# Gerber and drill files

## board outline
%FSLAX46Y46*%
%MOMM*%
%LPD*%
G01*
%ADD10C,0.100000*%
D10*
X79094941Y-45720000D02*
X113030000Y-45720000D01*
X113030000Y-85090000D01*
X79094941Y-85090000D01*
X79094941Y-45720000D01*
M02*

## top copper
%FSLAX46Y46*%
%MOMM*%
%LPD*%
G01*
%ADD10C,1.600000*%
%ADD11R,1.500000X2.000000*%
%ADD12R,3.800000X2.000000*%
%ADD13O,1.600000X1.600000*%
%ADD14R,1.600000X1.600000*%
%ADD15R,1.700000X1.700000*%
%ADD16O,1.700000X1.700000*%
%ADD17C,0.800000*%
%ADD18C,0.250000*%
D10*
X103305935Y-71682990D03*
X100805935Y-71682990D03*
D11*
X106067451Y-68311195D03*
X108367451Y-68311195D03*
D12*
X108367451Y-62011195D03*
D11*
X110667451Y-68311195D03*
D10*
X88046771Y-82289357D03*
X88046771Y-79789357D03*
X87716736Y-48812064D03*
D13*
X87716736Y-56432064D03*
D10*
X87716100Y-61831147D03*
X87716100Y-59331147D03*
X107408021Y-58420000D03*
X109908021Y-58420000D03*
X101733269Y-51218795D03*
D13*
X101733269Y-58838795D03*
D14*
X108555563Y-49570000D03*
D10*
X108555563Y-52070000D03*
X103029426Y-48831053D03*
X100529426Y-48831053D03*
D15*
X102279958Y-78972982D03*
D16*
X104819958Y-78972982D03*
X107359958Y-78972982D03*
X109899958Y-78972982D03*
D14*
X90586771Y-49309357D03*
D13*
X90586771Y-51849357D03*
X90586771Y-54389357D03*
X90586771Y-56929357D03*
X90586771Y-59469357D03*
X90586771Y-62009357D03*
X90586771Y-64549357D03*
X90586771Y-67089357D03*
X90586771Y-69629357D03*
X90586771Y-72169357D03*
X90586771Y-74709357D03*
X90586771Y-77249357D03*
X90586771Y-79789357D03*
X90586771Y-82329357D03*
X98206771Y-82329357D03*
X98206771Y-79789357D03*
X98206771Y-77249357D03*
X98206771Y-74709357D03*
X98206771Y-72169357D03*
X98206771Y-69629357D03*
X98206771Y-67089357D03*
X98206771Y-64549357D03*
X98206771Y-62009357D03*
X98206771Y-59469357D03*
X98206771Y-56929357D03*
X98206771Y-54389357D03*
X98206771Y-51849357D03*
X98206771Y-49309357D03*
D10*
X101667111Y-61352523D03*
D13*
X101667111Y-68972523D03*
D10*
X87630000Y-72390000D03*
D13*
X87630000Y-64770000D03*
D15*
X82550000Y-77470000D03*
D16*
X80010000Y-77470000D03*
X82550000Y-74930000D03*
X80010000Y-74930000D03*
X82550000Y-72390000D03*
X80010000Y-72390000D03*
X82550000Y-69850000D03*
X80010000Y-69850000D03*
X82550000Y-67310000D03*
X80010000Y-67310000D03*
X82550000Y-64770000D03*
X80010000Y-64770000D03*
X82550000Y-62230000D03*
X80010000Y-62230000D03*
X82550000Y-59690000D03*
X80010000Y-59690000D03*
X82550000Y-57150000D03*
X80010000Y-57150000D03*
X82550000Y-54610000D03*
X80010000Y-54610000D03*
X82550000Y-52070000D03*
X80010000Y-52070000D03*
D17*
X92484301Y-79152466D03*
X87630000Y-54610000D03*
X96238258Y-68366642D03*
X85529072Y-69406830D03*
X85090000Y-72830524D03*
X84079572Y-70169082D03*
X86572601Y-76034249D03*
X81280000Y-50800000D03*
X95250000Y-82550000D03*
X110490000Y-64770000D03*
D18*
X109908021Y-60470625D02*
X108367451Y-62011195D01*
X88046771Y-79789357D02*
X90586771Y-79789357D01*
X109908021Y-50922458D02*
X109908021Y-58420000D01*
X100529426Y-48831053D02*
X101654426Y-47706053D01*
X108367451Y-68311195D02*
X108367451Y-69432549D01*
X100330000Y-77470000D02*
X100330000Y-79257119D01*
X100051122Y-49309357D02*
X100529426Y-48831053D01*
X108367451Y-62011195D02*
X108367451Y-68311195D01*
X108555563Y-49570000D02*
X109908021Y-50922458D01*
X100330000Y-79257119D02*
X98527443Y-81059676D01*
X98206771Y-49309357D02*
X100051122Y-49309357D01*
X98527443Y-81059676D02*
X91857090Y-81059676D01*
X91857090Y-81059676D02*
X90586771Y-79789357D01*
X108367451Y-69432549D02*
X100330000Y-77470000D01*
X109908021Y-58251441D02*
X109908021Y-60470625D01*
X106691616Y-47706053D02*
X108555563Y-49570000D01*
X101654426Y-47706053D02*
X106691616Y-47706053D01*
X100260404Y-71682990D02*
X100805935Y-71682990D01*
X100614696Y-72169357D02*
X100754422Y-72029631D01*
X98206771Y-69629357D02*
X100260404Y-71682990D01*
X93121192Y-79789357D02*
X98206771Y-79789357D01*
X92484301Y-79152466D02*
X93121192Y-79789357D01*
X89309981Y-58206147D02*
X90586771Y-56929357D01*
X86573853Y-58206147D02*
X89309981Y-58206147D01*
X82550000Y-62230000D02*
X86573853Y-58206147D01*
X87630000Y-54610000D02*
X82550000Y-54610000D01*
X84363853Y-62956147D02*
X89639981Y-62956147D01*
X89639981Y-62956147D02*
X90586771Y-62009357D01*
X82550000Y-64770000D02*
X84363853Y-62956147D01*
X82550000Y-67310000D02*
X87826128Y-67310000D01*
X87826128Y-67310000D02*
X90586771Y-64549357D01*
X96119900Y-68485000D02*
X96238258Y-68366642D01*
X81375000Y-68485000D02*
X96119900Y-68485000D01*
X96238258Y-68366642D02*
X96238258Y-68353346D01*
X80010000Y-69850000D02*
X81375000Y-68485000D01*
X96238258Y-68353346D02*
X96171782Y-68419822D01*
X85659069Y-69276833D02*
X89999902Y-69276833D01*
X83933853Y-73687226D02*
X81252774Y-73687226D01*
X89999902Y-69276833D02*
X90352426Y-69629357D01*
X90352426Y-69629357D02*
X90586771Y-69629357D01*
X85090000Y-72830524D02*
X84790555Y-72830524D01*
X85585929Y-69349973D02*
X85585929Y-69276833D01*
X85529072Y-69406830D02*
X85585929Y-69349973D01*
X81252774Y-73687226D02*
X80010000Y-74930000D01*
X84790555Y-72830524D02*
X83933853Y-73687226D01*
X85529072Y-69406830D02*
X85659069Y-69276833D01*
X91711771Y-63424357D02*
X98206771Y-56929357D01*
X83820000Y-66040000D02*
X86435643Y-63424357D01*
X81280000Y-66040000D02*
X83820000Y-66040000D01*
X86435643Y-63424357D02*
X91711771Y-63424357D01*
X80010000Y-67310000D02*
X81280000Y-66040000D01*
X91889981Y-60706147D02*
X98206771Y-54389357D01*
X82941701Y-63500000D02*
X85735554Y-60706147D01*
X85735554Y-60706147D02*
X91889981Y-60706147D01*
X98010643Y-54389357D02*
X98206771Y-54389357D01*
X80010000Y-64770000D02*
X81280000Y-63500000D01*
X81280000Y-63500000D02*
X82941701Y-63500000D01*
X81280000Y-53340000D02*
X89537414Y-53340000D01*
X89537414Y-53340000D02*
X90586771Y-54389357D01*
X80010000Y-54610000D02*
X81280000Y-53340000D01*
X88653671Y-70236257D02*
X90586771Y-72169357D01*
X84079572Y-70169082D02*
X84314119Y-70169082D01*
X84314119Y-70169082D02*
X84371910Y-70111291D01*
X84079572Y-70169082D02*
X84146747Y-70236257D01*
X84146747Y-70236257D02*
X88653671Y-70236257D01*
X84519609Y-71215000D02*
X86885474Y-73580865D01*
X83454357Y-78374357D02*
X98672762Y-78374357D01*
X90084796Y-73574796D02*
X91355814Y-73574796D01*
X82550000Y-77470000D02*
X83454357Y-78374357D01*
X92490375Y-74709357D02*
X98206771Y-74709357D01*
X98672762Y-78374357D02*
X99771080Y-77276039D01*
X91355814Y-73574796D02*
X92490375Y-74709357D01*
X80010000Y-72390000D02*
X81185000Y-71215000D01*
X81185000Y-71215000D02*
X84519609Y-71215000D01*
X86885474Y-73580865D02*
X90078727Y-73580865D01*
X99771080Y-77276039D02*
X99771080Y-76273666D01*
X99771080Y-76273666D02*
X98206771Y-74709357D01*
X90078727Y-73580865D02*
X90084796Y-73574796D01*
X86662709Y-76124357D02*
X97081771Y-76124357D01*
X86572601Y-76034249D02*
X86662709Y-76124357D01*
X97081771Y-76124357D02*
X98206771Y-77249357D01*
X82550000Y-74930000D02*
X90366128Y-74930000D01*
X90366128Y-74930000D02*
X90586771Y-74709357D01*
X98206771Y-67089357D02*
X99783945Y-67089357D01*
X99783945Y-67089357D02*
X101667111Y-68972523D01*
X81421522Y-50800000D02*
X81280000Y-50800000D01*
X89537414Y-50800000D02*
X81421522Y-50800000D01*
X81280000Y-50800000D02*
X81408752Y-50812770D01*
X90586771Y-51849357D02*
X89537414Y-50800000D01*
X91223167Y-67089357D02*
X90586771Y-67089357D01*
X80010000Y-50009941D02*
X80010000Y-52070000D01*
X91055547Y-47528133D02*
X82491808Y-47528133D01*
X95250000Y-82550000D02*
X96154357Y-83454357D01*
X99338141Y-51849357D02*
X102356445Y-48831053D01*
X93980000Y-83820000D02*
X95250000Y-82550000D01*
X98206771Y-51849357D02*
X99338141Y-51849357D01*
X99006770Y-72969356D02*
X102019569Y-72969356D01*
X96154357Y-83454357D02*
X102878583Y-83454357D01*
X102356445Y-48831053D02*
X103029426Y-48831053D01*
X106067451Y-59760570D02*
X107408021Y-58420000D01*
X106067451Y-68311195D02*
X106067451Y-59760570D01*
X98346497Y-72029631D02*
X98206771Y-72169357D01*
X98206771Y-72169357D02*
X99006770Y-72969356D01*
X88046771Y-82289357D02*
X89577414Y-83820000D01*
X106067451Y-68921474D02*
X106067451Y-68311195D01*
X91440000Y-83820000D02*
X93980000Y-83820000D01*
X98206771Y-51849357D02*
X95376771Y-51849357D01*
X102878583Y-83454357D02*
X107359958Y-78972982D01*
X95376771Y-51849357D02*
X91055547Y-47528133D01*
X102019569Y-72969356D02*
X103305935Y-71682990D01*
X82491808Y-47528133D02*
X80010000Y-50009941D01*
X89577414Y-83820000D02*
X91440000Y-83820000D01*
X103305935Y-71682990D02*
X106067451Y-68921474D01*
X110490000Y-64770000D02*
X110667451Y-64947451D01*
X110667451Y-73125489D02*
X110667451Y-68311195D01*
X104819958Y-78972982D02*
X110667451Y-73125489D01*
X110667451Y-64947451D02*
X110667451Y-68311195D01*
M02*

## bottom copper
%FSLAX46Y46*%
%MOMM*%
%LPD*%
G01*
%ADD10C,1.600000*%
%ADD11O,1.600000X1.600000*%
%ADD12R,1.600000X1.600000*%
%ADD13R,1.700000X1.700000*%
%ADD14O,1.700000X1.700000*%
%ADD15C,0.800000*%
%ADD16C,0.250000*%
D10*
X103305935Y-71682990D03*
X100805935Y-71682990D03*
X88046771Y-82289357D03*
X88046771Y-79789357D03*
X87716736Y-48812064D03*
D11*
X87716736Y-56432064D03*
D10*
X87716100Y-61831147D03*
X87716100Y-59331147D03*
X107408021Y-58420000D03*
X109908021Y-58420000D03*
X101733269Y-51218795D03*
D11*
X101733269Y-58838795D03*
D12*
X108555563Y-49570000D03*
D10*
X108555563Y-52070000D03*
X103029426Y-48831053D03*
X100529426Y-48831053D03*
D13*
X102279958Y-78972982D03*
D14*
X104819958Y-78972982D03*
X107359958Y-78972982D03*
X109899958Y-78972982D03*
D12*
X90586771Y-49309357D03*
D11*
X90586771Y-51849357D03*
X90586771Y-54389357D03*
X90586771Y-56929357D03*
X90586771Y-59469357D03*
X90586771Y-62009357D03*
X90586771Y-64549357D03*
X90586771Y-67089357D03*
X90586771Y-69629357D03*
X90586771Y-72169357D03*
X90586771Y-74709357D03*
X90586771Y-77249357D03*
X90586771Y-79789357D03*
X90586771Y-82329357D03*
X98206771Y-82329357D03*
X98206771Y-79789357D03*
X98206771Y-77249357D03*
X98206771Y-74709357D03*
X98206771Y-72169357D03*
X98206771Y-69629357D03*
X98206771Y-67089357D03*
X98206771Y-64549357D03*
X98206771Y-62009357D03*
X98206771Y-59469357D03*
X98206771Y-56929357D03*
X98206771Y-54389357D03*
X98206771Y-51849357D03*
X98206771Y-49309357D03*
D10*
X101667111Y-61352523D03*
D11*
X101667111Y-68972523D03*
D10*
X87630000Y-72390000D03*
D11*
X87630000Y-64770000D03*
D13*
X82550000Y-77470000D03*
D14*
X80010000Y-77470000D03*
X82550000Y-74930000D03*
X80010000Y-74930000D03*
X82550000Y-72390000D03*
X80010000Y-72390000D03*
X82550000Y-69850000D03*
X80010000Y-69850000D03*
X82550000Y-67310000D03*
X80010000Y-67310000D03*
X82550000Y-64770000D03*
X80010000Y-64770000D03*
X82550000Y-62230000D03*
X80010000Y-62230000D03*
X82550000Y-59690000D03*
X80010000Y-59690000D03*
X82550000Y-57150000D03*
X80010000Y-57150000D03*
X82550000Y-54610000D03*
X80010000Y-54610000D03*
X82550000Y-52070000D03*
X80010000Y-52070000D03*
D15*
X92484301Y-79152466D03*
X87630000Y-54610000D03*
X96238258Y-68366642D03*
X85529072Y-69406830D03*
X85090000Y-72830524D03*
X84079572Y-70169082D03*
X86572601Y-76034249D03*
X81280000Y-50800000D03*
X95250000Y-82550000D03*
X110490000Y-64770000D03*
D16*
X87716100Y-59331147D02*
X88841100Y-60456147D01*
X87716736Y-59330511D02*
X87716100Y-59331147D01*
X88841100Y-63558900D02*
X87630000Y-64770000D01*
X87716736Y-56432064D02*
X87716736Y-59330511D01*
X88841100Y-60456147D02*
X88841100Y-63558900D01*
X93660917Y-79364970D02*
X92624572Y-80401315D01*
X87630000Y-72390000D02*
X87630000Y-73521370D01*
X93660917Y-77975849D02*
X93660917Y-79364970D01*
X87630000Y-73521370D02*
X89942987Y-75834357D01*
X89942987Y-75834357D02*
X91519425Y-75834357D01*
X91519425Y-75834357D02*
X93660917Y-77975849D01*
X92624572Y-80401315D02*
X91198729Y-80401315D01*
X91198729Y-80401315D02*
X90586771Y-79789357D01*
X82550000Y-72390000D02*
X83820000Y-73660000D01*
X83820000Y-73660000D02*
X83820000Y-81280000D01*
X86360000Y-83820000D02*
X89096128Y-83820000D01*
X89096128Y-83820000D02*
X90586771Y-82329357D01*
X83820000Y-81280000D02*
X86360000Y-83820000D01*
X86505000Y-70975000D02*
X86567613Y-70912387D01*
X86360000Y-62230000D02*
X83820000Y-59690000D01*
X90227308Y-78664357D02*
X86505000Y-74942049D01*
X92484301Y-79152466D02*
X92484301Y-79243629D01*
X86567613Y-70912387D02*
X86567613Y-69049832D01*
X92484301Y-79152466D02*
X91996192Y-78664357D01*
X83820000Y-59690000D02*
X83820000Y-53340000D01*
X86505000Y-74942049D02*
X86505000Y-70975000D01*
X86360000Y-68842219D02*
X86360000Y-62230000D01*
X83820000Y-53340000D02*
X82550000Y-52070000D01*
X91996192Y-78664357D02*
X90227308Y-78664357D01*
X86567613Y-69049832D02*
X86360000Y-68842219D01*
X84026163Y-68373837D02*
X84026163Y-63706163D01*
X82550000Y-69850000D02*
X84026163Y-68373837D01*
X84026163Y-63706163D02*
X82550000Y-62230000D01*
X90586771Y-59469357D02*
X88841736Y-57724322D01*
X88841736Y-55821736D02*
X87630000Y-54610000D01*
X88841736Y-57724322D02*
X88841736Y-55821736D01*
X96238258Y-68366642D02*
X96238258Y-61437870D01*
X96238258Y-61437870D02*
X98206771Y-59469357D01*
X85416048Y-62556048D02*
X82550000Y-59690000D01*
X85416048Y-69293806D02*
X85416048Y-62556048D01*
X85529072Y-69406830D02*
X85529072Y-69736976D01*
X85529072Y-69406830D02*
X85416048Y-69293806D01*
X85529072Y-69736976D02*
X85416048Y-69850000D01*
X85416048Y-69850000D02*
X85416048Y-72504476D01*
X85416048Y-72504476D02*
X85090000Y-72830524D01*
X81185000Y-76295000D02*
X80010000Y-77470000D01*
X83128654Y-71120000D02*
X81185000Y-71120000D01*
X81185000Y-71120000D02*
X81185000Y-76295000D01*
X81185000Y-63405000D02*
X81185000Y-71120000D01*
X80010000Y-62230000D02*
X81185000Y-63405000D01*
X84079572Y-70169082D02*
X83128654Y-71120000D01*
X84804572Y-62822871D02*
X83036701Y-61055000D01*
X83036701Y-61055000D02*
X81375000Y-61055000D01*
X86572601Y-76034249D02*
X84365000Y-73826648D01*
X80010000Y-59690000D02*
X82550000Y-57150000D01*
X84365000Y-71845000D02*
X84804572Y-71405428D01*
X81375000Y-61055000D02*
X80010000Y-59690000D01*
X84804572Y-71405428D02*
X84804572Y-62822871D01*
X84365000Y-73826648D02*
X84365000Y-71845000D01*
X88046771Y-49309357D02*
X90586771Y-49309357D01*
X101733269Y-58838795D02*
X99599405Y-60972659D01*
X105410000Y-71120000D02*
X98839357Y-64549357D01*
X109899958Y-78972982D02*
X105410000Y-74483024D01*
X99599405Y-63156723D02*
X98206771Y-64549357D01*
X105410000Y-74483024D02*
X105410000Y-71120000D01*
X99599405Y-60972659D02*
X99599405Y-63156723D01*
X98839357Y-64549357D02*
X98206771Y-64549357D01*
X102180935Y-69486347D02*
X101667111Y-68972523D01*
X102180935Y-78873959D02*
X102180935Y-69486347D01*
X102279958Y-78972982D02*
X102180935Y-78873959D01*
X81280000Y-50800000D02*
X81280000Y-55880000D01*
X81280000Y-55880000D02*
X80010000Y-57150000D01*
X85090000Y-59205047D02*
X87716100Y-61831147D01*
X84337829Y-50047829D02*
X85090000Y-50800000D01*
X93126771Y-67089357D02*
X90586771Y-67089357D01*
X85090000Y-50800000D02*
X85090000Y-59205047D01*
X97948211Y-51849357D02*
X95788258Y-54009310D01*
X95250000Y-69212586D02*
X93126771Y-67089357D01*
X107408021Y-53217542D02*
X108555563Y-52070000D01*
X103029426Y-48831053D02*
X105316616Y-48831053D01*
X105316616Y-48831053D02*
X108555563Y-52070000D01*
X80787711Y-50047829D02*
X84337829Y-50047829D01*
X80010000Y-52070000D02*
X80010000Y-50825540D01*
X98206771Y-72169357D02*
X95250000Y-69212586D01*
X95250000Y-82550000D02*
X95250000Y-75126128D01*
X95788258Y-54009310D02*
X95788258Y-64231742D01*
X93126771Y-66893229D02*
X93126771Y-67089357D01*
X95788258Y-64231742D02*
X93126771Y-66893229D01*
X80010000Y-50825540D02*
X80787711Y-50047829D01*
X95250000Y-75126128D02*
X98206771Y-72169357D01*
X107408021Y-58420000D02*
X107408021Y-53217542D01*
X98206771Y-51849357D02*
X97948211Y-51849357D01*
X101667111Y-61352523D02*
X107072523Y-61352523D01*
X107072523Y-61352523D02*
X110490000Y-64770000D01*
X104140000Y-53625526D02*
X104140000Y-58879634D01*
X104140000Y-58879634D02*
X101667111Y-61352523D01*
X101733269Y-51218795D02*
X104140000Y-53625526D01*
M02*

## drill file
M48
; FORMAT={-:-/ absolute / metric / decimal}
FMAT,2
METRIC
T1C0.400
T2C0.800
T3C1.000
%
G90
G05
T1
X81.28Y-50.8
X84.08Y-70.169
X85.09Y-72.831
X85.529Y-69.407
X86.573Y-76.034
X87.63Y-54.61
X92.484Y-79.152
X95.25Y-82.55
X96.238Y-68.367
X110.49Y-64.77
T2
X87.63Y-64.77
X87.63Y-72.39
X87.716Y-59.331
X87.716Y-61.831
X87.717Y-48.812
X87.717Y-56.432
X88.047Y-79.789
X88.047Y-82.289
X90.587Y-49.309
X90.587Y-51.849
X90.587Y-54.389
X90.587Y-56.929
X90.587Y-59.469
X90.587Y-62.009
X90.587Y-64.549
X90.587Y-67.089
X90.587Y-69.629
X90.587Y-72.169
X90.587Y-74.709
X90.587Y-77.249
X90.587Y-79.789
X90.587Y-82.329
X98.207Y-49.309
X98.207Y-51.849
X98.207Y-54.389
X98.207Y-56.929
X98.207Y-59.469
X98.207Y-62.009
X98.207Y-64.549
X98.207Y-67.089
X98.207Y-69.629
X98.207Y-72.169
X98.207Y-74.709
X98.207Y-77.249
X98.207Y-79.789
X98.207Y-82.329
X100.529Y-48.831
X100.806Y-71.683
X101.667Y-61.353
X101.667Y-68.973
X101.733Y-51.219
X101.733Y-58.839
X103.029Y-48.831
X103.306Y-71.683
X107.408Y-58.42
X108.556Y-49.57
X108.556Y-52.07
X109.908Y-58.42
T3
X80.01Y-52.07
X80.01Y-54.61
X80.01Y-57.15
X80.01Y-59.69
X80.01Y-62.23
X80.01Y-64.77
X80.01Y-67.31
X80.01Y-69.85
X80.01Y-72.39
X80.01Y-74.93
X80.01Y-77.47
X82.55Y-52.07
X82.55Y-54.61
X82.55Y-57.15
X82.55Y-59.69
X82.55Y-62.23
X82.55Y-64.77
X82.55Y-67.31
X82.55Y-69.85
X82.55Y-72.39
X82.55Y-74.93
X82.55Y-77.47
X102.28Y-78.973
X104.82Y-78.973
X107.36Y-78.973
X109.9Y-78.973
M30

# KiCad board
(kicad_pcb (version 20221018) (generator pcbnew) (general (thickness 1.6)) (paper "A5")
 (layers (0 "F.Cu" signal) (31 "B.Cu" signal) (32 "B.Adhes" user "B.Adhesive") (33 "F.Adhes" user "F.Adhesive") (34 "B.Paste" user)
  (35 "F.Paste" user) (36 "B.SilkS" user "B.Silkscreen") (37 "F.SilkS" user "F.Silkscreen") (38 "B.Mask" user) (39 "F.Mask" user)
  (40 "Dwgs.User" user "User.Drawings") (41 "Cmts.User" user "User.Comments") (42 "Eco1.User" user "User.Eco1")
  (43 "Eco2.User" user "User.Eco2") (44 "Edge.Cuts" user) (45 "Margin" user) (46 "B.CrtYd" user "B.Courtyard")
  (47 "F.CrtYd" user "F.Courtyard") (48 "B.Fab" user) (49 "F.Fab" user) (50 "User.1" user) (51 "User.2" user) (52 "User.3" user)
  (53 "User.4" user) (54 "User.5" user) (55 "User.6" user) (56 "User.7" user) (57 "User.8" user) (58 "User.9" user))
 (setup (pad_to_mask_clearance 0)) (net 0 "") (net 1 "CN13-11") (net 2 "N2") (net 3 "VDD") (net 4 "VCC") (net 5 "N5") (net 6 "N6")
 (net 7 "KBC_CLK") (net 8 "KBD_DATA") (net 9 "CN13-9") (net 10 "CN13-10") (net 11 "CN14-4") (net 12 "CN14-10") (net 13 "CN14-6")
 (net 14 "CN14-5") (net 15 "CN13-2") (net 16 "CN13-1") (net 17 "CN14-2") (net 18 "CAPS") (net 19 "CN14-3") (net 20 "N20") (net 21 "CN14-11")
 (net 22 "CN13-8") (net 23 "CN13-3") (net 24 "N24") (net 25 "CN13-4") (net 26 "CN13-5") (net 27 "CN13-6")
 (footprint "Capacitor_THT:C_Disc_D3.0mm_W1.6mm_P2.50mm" (layer "F.Cu") (at 103.305935 71.68299 180)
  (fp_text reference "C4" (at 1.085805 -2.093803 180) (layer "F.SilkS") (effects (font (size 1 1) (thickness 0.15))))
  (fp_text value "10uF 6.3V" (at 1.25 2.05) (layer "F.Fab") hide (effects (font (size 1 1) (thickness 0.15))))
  (pad "1" thru_hole circle (at 0 0 180) (size 1.6 1.6) (drill 0.8) (layers "*.Cu" "*.Mask") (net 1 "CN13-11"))
  (pad "2" thru_hole circle (at 2.5 0 180) (size 1.6 1.6) (drill 0.8) (layers "*.Cu" "*.Mask") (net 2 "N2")))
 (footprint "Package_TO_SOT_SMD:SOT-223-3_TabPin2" (layer "F.Cu") (at 108.367451 65.161195 90)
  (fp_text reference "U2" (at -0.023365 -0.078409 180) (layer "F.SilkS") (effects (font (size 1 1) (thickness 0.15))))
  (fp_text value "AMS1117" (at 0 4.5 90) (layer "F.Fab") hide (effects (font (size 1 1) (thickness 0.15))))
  (pad "1" smd rect (at -3.15 -2.3 90) (size 2 1.5) (layers "F.Cu" "F.Paste" "F.Mask") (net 1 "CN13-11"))
  (pad "2" smd rect (at -3.15 0 90) (size 2 1.5) (layers "F.Cu" "F.Paste" "F.Mask") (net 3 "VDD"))
  (pad "2" smd rect (at 3.15 0 90) (size 2 3.8) (layers "F.Cu" "F.Paste" "F.Mask") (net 3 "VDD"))
  (pad "3" smd rect (at -3.15 2.3 90) (size 2 1.5) (layers "F.Cu" "F.Paste" "F.Mask") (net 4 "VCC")))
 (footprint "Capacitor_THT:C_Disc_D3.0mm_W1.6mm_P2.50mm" (layer "F.Cu") (at 88.046771 82.289357 90)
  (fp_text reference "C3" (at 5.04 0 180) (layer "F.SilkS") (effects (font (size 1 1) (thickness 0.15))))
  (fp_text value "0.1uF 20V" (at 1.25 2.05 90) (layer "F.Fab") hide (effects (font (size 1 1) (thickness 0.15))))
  (pad "1" thru_hole circle (at 0 0 90) (size 1.6 1.6) (drill 0.8) (layers "*.Cu" "*.Mask") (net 1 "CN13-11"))
  (pad "2" thru_hole circle (at 2.5 0 90) (size 1.6 1.6) (drill 0.8) (layers "*.Cu" "*.Mask") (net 3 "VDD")))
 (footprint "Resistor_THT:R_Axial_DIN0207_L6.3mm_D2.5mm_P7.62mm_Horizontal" (layer "F.Cu") (at 87.716736 48.812064 -90)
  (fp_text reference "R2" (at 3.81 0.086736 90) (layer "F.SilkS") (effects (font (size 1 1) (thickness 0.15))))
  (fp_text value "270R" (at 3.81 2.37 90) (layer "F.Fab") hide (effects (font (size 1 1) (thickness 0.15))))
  (pad "1" thru_hole circle (at 0 0 270) (size 1.6 1.6) (drill 0.8) (layers "*.Cu" "*.Mask") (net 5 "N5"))
  (pad "2" thru_hole oval (at 7.62 0 270) (size 1.6 1.6) (drill 0.8) (layers "*.Cu" "*.Mask") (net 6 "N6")))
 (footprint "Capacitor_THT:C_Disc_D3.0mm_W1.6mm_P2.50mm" (layer "F.Cu") (at 87.7161 61.831147 90)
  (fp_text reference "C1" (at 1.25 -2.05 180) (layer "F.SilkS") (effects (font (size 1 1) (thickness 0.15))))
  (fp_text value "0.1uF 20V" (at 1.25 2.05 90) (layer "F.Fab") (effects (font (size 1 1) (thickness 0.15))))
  (pad "1" thru_hole circle (at 0 0 90) (size 1.6 1.6) (drill 0.8) (layers "*.Cu" "*.Mask") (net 1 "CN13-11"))
  (pad "2" thru_hole circle (at 2.5 0 90) (size 1.6 1.6) (drill 0.8) (layers "*.Cu" "*.Mask") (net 6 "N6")))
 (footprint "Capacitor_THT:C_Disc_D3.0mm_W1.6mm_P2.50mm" (layer "F.Cu") (at 107.408021 58.42)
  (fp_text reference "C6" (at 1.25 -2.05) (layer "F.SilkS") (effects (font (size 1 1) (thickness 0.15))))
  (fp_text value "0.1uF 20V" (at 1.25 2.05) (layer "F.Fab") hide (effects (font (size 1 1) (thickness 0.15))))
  (pad "1" thru_hole circle (at 0 0) (size 1.6 1.6) (drill 0.8) (layers "*.Cu" "*.Mask") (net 1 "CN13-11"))
  (pad "2" thru_hole circle (at 2.5 0) (size 1.6 1.6) (drill 0.8) (layers "*.Cu" "*.Mask") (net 3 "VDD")))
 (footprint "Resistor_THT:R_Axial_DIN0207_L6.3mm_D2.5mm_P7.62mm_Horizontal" (layer "F.Cu") (at 101.733269 51.218795 -90)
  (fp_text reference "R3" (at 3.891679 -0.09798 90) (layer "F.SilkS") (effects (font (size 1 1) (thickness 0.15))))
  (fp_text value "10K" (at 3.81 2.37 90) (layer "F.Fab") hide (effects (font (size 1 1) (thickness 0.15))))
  (pad "1" thru_hole circle (at 0 0 270) (size 1.6 1.6) (drill 0.8) (layers "*.Cu" "*.Mask") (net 4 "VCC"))
  (pad "2" thru_hole oval (at 7.62 0 270) (size 1.6 1.6) (drill 0.8) (layers "*.Cu" "*.Mask") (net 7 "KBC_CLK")))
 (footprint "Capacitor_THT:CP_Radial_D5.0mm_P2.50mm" (layer "F.Cu") (at 108.555563 49.57 -90)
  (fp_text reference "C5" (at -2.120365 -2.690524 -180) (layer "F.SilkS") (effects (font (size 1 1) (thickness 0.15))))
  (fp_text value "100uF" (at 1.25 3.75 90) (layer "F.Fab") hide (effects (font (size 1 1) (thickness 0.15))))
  (pad "1" thru_hole rect (at 0 0 270) (size 1.6 1.6) (drill 0.8) (layers "*.Cu" "*.Mask") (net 3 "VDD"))
  (pad "2" thru_hole circle (at 2.5 0 270) (size 1.6 1.6) (drill 0.8) (layers "*.Cu" "*.Mask") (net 1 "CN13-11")))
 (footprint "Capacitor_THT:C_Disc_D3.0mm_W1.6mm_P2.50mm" (layer "F.Cu") (at 103.029426 48.831053 180)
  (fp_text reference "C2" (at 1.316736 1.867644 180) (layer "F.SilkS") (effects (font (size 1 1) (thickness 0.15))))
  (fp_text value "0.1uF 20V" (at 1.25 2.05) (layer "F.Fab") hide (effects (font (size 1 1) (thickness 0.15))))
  (pad "1" thru_hole circle (at 0 0 180) (size 1.6 1.6) (drill 0.8) (layers "*.Cu" "*.Mask") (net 1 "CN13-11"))
  (pad "2" thru_hole circle (at 2.5 0 180) (size 1.6 1.6) (drill 0.8) (layers "*.Cu" "*.Mask") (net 3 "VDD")))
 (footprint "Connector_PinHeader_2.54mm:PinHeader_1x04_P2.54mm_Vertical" (layer "F.Cu") (at 102.279958 78.972982 90)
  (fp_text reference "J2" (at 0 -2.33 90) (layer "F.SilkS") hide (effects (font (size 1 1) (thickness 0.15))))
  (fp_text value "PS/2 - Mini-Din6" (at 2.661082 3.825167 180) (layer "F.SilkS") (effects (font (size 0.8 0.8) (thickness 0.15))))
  (pad "1" thru_hole rect (at 0 0 90) (size 1.7 1.7) (drill 1) (layers "*.Cu" "*.Mask") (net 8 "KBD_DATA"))
  (pad "2" thru_hole oval (at 0 2.54 90) (size 1.7 1.7) (drill 1) (layers "*.Cu" "*.Mask") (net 4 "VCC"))
  (pad "3" thru_hole oval (at 0 5.08 90) (size 1.7 1.7) (drill 1) (layers "*.Cu" "*.Mask") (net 1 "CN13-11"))
  (pad "4" thru_hole oval (at 0 7.62 90) (size 1.7 1.7) (drill 1) (layers "*.Cu" "*.Mask") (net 7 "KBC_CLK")))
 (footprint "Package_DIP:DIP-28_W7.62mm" (layer "F.Cu") (at 90.586771 49.309357)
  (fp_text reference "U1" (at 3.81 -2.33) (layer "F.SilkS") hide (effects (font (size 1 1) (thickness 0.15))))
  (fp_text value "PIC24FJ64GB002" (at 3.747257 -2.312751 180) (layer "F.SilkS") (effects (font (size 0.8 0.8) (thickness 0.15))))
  (pad "1" thru_hole rect (at 0 0) (size 1.6 1.6) (drill 0.8) (layers "*.Cu" "*.Mask") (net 5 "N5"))
  (pad "2" thru_hole oval (at 0 2.54) (size 1.6 1.6) (drill 0.8) (layers "*.Cu" "*.Mask") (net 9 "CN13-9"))
  (pad "3" thru_hole oval (at 0 5.08) (size 1.6 1.6) (drill 0.8) (layers "*.Cu" "*.Mask") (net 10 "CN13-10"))
  (pad "4" thru_hole oval (at 0 7.62) (size 1.6 1.6) (drill 0.8) (layers "*.Cu" "*.Mask") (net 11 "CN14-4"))
  (pad "5" thru_hole oval (at 0 10.16) (size 1.6 1.6) (drill 0.8) (layers "*.Cu" "*.Mask") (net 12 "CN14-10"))
  (pad "6" thru_hole oval (at 0 12.7) (size 1.6 1.6) (drill 0.8) (layers "*.Cu" "*.Mask") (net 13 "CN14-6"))
  (pad "7" thru_hole oval (at 0 15.24) (size 1.6 1.6) (drill 0.8) (layers "*.Cu" "*.Mask") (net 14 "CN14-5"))
  (pad "8" thru_hole oval (at 0 17.78) (size 1.6 1.6) (drill 0.8) (layers "*.Cu" "*.Mask") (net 1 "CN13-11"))
  (pad "9" thru_hole oval (at 0 20.32) (size 1.6 1.6) (drill 0.8) (layers "*.Cu" "*.Mask") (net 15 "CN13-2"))
  (pad "10" thru_hole oval (at 0 22.86) (size 1.6 1.6) (drill 0.8) (layers "*.Cu" "*.Mask") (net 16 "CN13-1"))
  (pad "11" thru_hole oval (at 0 25.4) (size 1.6 1.6) (drill 0.8) (layers "*.Cu" "*.Mask") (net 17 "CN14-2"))
  (pad "12" thru_hole oval (at 0 27.94) (size 1.6 1.6) (drill 0.8) (layers "*.Cu" "*.Mask") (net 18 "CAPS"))
  (pad "13" thru_hole oval (at 0 30.48) (size 1.6 1.6) (drill 0.8) (layers "*.Cu" "*.Mask") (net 3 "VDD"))
  (pad "14" thru_hole oval (at 0 33.02) (size 1.6 1.6) (drill 0.8) (layers "*.Cu" "*.Mask") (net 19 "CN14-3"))
  (pad "15" thru_hole oval (at 7.62 33.02) (size 1.6 1.6) (drill 0.8) (layers "*.Cu" "*.Mask") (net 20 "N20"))
  (pad "16" thru_hole oval (at 7.62 30.48) (size 1.6 1.6) (drill 0.8) (layers "*.Cu" "*.Mask") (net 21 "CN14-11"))
  (pad "17" thru_hole oval (at 7.62 27.94) (size 1.6 1.6) (drill 0.8) (layers "*.Cu" "*.Mask") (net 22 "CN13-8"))
  (pad "18" thru_hole oval (at 7.62 25.4) (size 1.6 1.6) (drill 0.8) (layers "*.Cu" "*.Mask") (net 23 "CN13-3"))
  (pad "19" thru_hole oval (at 7.62 22.86) (size 1.6 1.6) (drill 0.8) (layers "*.Cu" "*.Mask") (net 1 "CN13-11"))
  (pad "20" thru_hole oval (at 7.62 20.32) (size 1.6 1.6) (drill 0.8) (layers "*.Cu" "*.Mask") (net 2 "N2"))
  (pad "21" thru_hole oval (at 7.62 17.78) (size 1.6 1.6) (drill 0.8) (layers "*.Cu" "*.Mask") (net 8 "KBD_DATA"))
  (pad "22" thru_hole oval (at 7.62 15.24) (size 1.6 1.6) (drill 0.8) (layers "*.Cu" "*.Mask") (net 7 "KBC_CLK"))
  (pad "23" thru_hole oval (at 7.62 12.7) (size 1.6 1.6) (drill 0.8) (layers "*.Cu" "*.Mask") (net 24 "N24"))
  (pad "24" thru_hole oval (at 7.62 10.16) (size 1.6 1.6) (drill 0.8) (layers "*.Cu" "*.Mask") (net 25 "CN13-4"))
  (pad "25" thru_hole oval (at 7.62 7.62) (size 1.6 1.6) (drill 0.8) (layers "*.Cu" "*.Mask") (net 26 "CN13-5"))
  (pad "26" thru_hole oval (at 7.62 5.08) (size 1.6 1.6) (drill 0.8) (layers "*.Cu" "*.Mask") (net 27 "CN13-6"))
  (pad "27" thru_hole oval (at 7.62 2.54) (size 1.6 1.6) (drill 0.8) (layers "*.Cu" "*.Mask") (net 1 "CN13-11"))
  (pad "28" thru_hole oval (at 7.62 0) (size 1.6 1.6) (drill 0.8) (layers "*.Cu" "*.Mask") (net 3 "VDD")))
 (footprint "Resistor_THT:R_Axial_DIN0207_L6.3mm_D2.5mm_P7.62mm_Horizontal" (layer "F.Cu") (at 101.667111 61.352523 -90)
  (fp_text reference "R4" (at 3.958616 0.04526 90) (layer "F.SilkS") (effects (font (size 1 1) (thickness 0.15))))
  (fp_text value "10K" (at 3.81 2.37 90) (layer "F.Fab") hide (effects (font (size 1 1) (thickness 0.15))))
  (pad "1" thru_hole circle (at 0 0 270) (size 1.6 1.6) (drill 0.8) (layers "*.Cu" "*.Mask") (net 4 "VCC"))
  (pad "2" thru_hole oval (at 7.62 0 270) (size 1.6 1.6) (drill 0.8) (layers "*.Cu" "*.Mask") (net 8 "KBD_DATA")))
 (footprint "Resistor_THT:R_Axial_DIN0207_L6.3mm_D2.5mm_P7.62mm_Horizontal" (layer "F.Cu") (at 87.63 72.39 90)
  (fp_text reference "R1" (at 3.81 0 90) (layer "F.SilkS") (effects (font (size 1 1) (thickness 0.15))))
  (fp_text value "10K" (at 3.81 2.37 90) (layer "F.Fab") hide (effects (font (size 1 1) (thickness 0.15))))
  (pad "1" thru_hole circle (at 0 0 90) (size 1.6 1.6) (drill 0.8) (layers "*.Cu" "*.Mask") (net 3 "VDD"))
  (pad "2" thru_hole oval (at 7.62 0 90) (size 1.6 1.6) (drill 0.8) (layers "*.Cu" "*.Mask") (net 6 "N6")))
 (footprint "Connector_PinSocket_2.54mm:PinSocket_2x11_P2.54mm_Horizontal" (layer "B.Cu") (at 82.55 77.47)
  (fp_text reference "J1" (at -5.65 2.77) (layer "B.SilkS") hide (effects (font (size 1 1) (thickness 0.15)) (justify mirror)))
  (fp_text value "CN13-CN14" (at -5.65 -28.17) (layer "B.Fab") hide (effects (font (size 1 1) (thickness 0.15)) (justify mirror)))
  (pad "1" thru_hole rect (at 0 0) (size 1.7 1.7) (drill 1) (layers "*.Cu" "*.Mask") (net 23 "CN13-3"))
  (pad "2" thru_hole oval (at -2.54 0) (size 1.7 1.7) (drill 1) (layers "*.Cu" "*.Mask") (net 16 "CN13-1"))
  (pad "3" thru_hole oval (at 0 -2.54) (size 1.7 1.7) (drill 1) (layers "*.Cu" "*.Mask") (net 17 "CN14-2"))
  (pad "4" thru_hole oval (at -2.54 -2.54) (size 1.7 1.7) (drill 1) (layers "*.Cu" "*.Mask") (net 15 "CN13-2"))
  (pad "5" thru_hole oval (at 0 -5.08) (size 1.7 1.7) (drill 1) (layers "*.Cu" "*.Mask") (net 19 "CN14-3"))
  (pad "6" thru_hole oval (at -2.54 -5.08) (size 1.7 1.7) (drill 1) (layers "*.Cu" "*.Mask") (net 23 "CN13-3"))
  (pad "7" thru_hole oval (at 0 -7.62) (size 1.7 1.7) (drill 1) (layers "*.Cu" "*.Mask") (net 11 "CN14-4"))
  (pad "8" thru_hole oval (at -2.54 -7.62) (size 1.7 1.7) (drill 1) (layers "*.Cu" "*.Mask") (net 25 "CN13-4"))
  (pad "9" thru_hole oval (at 0 -10.16) (size 1.7 1.7) (drill 1) (layers "*.Cu" "*.Mask") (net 14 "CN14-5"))
  (pad "10" thru_hole oval (at -2.54 -10.16) (size 1.7 1.7) (drill 1) (layers "*.Cu" "*.Mask") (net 26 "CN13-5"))
  (pad "11" thru_hole oval (at 0 -12.7) (size 1.7 1.7) (drill 1) (layers "*.Cu" "*.Mask") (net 13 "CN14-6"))
  (pad "12" thru_hole oval (at -2.54 -12.7) (size 1.7 1.7) (drill 1) (layers "*.Cu" "*.Mask") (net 27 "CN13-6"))
  (pad "13" thru_hole oval (at 0 -15.24) (size 1.7 1.7) (drill 1) (layers "*.Cu" "*.Mask") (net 11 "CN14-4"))
  (pad "14" thru_hole oval (at -2.54 -15.24) (size 1.7 1.7) (drill 1) (layers "*.Cu" "*.Mask") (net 16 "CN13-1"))
  (pad "15" thru_hole oval (at 0 -17.78) (size 1.7 1.7) (drill 1) (layers "*.Cu" "*.Mask") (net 15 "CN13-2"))
  (pad "16" thru_hole oval (at -2.54 -17.78) (size 1.7 1.7) (drill 1) (layers "*.Cu" "*.Mask") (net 22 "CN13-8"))
  (pad "17" thru_hole oval (at 0 -20.32) (size 1.7 1.7) (drill 1) (layers "*.Cu" "*.Mask") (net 22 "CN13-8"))
  (pad "18" thru_hole oval (at -2.54 -20.32) (size 1.7 1.7) (drill 1) (layers "*.Cu" "*.Mask") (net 9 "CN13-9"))
  (pad "19" thru_hole oval (at 0 -22.86) (size 1.7 1.7) (drill 1) (layers "*.Cu" "*.Mask") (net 12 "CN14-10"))
  (pad "20" thru_hole oval (at -2.54 -22.86) (size 1.7 1.7) (drill 1) (layers "*.Cu" "*.Mask") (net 10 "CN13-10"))
  (pad "21" thru_hole oval (at 0 -25.4) (size 1.7 1.7) (drill 1) (layers "*.Cu" "*.Mask") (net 21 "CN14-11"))
  (pad "22" thru_hole oval (at -2.54 -25.4) (size 1.7 1.7) (drill 1) (layers "*.Cu" "*.Mask") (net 1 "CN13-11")))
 (gr_rect (start 79.094941 45.72) (end 113.03 85.09) (stroke (width 0.1) (type default)) (fill none) (layer "Edge.Cuts"))
 (segment (start 87.7161 59.331147) (end 88.8411 60.456147) (width 0.25) (layer "B.Cu") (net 6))
 (segment (start 87.716736 59.330511) (end 87.7161 59.331147) (width 0.25) (layer "B.Cu") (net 6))
 (segment (start 88.8411 63.5589) (end 87.63 64.77) (width 0.25) (layer "B.Cu") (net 6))
 (segment (start 87.716736 56.432064) (end 87.716736 59.330511) (width 0.25) (layer "B.Cu") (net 6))
 (segment (start 88.8411 60.456147) (end 88.8411 63.5589) (width 0.25) (layer "B.Cu") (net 6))
 (segment (start 109.908021 60.470625) (end 108.367451 62.011195) (width 0.25) (layer "F.Cu") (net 3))
 (segment (start 88.046771 79.789357) (end 90.586771 79.789357) (width 0.25) (layer "F.Cu") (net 3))
 (segment (start 109.908021 50.922458) (end 109.908021 58.42) (width 0.25) (layer "F.Cu") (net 3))
 (segment (start 100.529426 48.831053) (end 101.654426 47.706053) (width 0.25) (layer "F.Cu") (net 3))
 (segment (start 108.367451 68.311195) (end 108.367451 69.432549) (width 0.25) (layer "F.Cu") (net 3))
 (segment (start 100.33 77.47) (end 100.33 79.257119) (width 0.25) (layer "F.Cu") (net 3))
 (segment (start 100.051122 49.309357) (end 100.529426 48.831053) (width 0.25) (layer "F.Cu") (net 3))
 (segment (start 108.367451 62.011195) (end 108.367451 68.311195) (width 0.25) (layer "F.Cu") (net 3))
 (segment (start 108.555563 49.57) (end 109.908021 50.922458) (width 0.25) (layer "F.Cu") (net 3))
 (segment (start 100.33 79.257119) (end 98.527443 81.059676) (width 0.25) (layer "F.Cu") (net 3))
 (segment (start 98.206771 49.309357) (end 100.051122 49.309357) (width 0.25) (layer "F.Cu") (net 3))
 (segment (start 98.527443 81.059676) (end 91.85709 81.059676) (width 0.25) (layer "F.Cu") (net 3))
 (segment (start 91.85709 81.059676) (end 90.586771 79.789357) (width 0.25) (layer "F.Cu") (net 3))
 (segment (start 108.367451 69.432549) (end 100.33 77.47) (width 0.25) (layer "F.Cu") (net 3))
 (segment (start 109.908021 58.251441) (end 109.908021 60.470625) (width 0.25) (layer "F.Cu") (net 3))
 (segment (start 106.691616 47.706053) (end 108.555563 49.57) (width 0.25) (layer "F.Cu") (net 3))
 (segment (start 101.654426 47.706053) (end 106.691616 47.706053) (width 0.25) (layer "F.Cu") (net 3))
 (segment (start 93.660917 79.36497) (end 92.624572 80.401315) (width 0.25) (layer "B.Cu") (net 3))
 (segment (start 87.63 72.39) (end 87.63 73.52137) (width 0.25) (layer "B.Cu") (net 3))
 (segment (start 93.660917 77.975849) (end 93.660917 79.36497) (width 0.25) (layer "B.Cu") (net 3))
 (segment (start 87.63 73.52137) (end 89.942987 75.834357) (width 0.25) (layer "B.Cu") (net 3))
 (segment (start 89.942987 75.834357) (end 91.519425 75.834357) (width 0.25) (layer "B.Cu") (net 3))
 (segment (start 91.519425 75.834357) (end 93.660917 77.975849) (width 0.25) (layer "B.Cu") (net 3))
 (segment (start 92.624572 80.401315) (end 91.198729 80.401315) (width 0.25) (layer "B.Cu") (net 3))
 (segment (start 91.198729 80.401315) (end 90.586771 79.789357) (width 0.25) (layer "B.Cu") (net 3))
 (segment (start 100.260404 71.68299) (end 100.805935 71.68299) (width 0.25) (layer "F.Cu") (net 2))
 (segment (start 100.614696 72.169357) (end 100.754422 72.029631) (width 0.25) (layer "F.Cu") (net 2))
 (segment (start 98.206771 69.629357) (end 100.260404 71.68299) (width 0.25) (layer "F.Cu") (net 2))
 (segment (start 82.55 72.39) (end 83.82 73.66) (width 0.25) (layer "B.Cu") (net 19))
 (segment (start 83.82 73.66) (end 83.82 81.28) (width 0.25) (layer "B.Cu") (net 19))
 (segment (start 86.36 83.82) (end 89.096128 83.82) (width 0.25) (layer "B.Cu") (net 19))
 (segment (start 89.096128 83.82) (end 90.586771 82.329357) (width 0.25) (layer "B.Cu") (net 19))
 (segment (start 83.82 81.28) (end 86.36 83.82) (width 0.25) (layer "B.Cu") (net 19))
 (segment (start 93.121192 79.789357) (end 98.206771 79.789357) (width 0.25) (layer "F.Cu") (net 21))
 (segment (start 92.484301 79.152466) (end 93.121192 79.789357) (width 0.25) (layer "F.Cu") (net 21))
 (via (at 92.484301 79.152466) (size 0.8) (drill 0.4) (layers "F.Cu" "B.Cu") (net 21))
 (segment (start 86.505 70.975) (end 86.567613 70.912387) (width 0.25) (layer "B.Cu") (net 21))
 (segment (start 86.36 62.23) (end 83.82 59.69) (width 0.25) (layer "B.Cu") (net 21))
 (segment (start 90.227308 78.664357) (end 86.505 74.942049) (width 0.25) (layer "B.Cu") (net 21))
 (segment (start 92.484301 79.152466) (end 92.484301 79.243629) (width 0.25) (layer "B.Cu") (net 21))
 (segment (start 86.567613 70.912387) (end 86.567613 69.049832) (width 0.25) (layer "B.Cu") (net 21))
 (segment (start 92.484301 79.152466) (end 91.996192 78.664357) (width 0.25) (layer "B.Cu") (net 21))
 (segment (start 83.82 59.69) (end 83.82 53.34) (width 0.25) (layer "B.Cu") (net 21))
 (segment (start 86.505 74.942049) (end 86.505 70.975) (width 0.25) (layer "B.Cu") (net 21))
 (segment (start 86.36 68.842219) (end 86.36 62.23) (width 0.25) (layer "B.Cu") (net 21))
 (segment (start 83.82 53.34) (end 82.55 52.07) (width 0.25) (layer "B.Cu") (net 21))
 (segment (start 91.996192 78.664357) (end 90.227308 78.664357) (width 0.25) (layer "B.Cu") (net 21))
 (segment (start 86.567613 69.049832) (end 86.36 68.842219) (width 0.25) (layer "B.Cu") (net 21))
 (segment (start 89.309981 58.206147) (end 90.586771 56.929357) (width 0.25) (layer "F.Cu") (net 11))
 (segment (start 86.573853 58.206147) (end 89.309981 58.206147) (width 0.25) (layer "F.Cu") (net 11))
 (segment (start 82.55 62.23) (end 86.573853 58.206147) (width 0.25) (layer "F.Cu") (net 11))
 (segment (start 84.026163 68.373837) (end 84.026163 63.706163) (width 0.25) (layer "B.Cu") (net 11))
 (segment (start 82.55 69.85) (end 84.026163 68.373837) (width 0.25) (layer "B.Cu") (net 11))
 (segment (start 84.026163 63.706163) (end 82.55 62.23) (width 0.25) (layer "B.Cu") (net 11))
 (segment (start 87.63 54.61) (end 82.55 54.61) (width 0.25) (layer "F.Cu") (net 12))
 (via (at 87.63 54.61) (size 0.8) (drill 0.4) (layers "F.Cu" "B.Cu") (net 12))
 (segment (start 90.586771 59.469357) (end 88.841736 57.724322) (width 0.25) (layer "B.Cu") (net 12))
 (segment (start 88.841736 55.821736) (end 87.63 54.61) (width 0.25) (layer "B.Cu") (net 12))
 (segment (start 88.841736 57.724322) (end 88.841736 55.821736) (width 0.25) (layer "B.Cu") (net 12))
 (segment (start 84.363853 62.956147) (end 89.639981 62.956147) (width 0.25) (layer "F.Cu") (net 13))
 (segment (start 89.639981 62.956147) (end 90.586771 62.009357) (width 0.25) (layer "F.Cu") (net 13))
 (segment (start 82.55 64.77) (end 84.363853 62.956147) (width 0.25) (layer "F.Cu") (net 13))
 (segment (start 82.55 67.31) (end 87.826128 67.31) (width 0.25) (layer "F.Cu") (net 14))
 (segment (start 87.826128 67.31) (end 90.586771 64.549357) (width 0.25) (layer "F.Cu") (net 14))
 (segment (start 96.1199 68.485) (end 96.238258 68.366642) (width 0.25) (layer "F.Cu") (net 25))
 (segment (start 81.375 68.485) (end 96.1199 68.485) (width 0.25) (layer "F.Cu") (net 25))
 (segment (start 96.238258 68.366642) (end 96.238258 68.353346) (width 0.25) (layer "F.Cu") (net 25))
 (segment (start 80.01 69.85) (end 81.375 68.485) (width 0.25) (layer "F.Cu") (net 25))
 (segment (start 96.238258 68.353346) (end 96.171782 68.419822) (width 0.25) (layer "F.Cu") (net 25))
 (via (at 96.238258 68.366642) (size 0.8) (drill 0.4) (layers "F.Cu" "B.Cu") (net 25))
 (segment (start 96.238258 68.366642) (end 96.238258 61.43787) (width 0.25) (layer "B.Cu") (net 25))
 (segment (start 96.238258 61.43787) (end 98.206771 59.469357) (width 0.25) (layer "B.Cu") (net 25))
 (segment (start 85.659069 69.276833) (end 89.999902 69.276833) (width 0.25) (layer "F.Cu") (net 15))
 (segment (start 83.933853 73.687226) (end 81.252774 73.687226) (width 0.25) (layer "F.Cu") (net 15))
 (segment (start 89.999902 69.276833) (end 90.352426 69.629357) (width 0.25) (layer "F.Cu") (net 15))
 (segment (start 90.352426 69.629357) (end 90.586771 69.629357) (width 0.25) (layer "F.Cu") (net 15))
 (segment (start 85.09 72.830524) (end 84.790555 72.830524) (width 0.25) (layer "F.Cu") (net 15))
 (segment (start 85.585929 69.349973) (end 85.585929 69.276833) (width 0.25) (layer "F.Cu") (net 15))
 (segment (start 85.529072 69.40683) (end 85.585929 69.349973) (width 0.25) (layer "F.Cu") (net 15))
 (segment (start 81.252774 73.687226) (end 80.01 74.93) (width 0.25) (layer "F.Cu") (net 15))
 (segment (start 84.790555 72.830524) (end 83.933853 73.687226) (width 0.25) (layer "F.Cu") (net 15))
 (segment (start 85.529072 69.40683) (end 85.659069 69.276833) (width 0.25) (layer "F.Cu") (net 15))
 (via (at 85.529072 69.40683) (size 0.8) (drill 0.4) (layers "F.Cu" "B.Cu") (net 15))
 (via (at 85.09 72.830524) (size 0.8) (drill 0.4) (layers "F.Cu" "B.Cu") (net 15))
 (segment (start 85.416048 62.556048) (end 82.55 59.69) (width 0.25) (layer "B.Cu") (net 15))
 (segment (start 85.416048 69.293806) (end 85.416048 62.556048) (width 0.25) (layer "B.Cu") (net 15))
 (segment (start 85.529072 69.40683) (end 85.529072 69.736976) (width 0.25) (layer "B.Cu") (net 15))
 (segment (start 85.529072 69.40683) (end 85.416048 69.293806) (width 0.25) (layer "B.Cu") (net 15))
 (segment (start 85.529072 69.736976) (end 85.416048 69.85) (width 0.25) (layer "B.Cu") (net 15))
 (segment (start 85.416048 69.85) (end 85.416048 72.504476) (width 0.25) (layer "B.Cu") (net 15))
 (segment (start 85.416048 72.504476) (end 85.09 72.830524) (width 0.25) (layer "B.Cu") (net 15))
 (segment (start 91.711771 63.424357) (end 98.206771 56.929357) (width 0.25) (layer "F.Cu") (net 26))
 (segment (start 83.82 66.04) (end 86.435643 63.424357) (width 0.25) (layer "F.Cu") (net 26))
 (segment (start 81.28 66.04) (end 83.82 66.04) (width 0.25) (layer "F.Cu") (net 26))
 (segment (start 86.435643 63.424357) (end 91.711771 63.424357) (width 0.25) (layer "F.Cu") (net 26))
 (segment (start 80.01 67.31) (end 81.28 66.04) (width 0.25) (layer "F.Cu") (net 26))
 (segment (start 91.889981 60.706147) (end 98.206771 54.389357) (width 0.25) (layer "F.Cu") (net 27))
 (segment (start 82.941701 63.5) (end 85.735554 60.706147) (width 0.25) (layer "F.Cu") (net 27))
 (segment (start 85.735554 60.706147) (end 91.889981 60.706147) (width 0.25) (layer "F.Cu") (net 27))
 (segment (start 98.010643 54.389357) (end 98.206771 54.389357) (width 0.25) (layer "F.Cu") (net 27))
 (segment (start 80.01 64.77) (end 81.28 63.5) (width 0.25) (layer "F.Cu") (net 27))
 (segment (start 81.28 63.5) (end 82.941701 63.5) (width 0.25) (layer "F.Cu") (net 27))
 (segment (start 81.28 53.34) (end 89.537414 53.34) (width 0.25) (layer "F.Cu") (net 10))
 (segment (start 89.537414 53.34) (end 90.586771 54.389357) (width 0.25) (layer "F.Cu") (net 10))
 (segment (start 80.01 54.61) (end 81.28 53.34) (width 0.25) (layer "F.Cu") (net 10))
 (segment (start 88.653671 70.236257) (end 90.586771 72.169357) (width 0.25) (layer "F.Cu") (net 16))
 (segment (start 84.079572 70.169082) (end 84.314119 70.169082) (width 0.25) (layer "F.Cu") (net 16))
 (segment (start 84.314119 70.169082) (end 84.37191 70.111291) (width 0.25) (layer "F.Cu") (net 16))
 (segment (start 84.079572 70.169082) (end 84.146747 70.236257) (width 0.25) (layer "F.Cu") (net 16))
 (segment (start 84.146747 70.236257) (end 88.653671 70.236257) (width 0.25) (layer "F.Cu") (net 16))
 (via (at 84.079572 70.169082) (size 0.8) (drill 0.4) (layers "F.Cu" "B.Cu") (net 16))
 (segment (start 81.185 76.295) (end 80.01 77.47) (width 0.25) (layer "B.Cu") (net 16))
 (segment (start 83.128654 71.12) (end 81.185 71.12) (width 0.25) (layer "B.Cu") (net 16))
 (segment (start 81.185 71.12) (end 81.185 76.295) (width 0.25) (layer "B.Cu") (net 16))
 (segment (start 81.185 63.405) (end 81.185 71.12) (width 0.25) (layer "B.Cu") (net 16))
 (segment (start 80.01 62.23) (end 81.185 63.405) (width 0.25) (layer "B.Cu") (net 16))
 (segment (start 84.079572 70.169082) (end 83.128654 71.12) (width 0.25) (layer "B.Cu") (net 16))
 (segment (start 84.519609 71.215) (end 86.885474 73.580865) (width 0.25) (layer "F.Cu") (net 23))
 (segment (start 83.454357 78.374357) (end 98.672762 78.374357) (width 0.25) (layer "F.Cu") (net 23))
 (segment (start 90.084796 73.574796) (end 91.355814 73.574796) (width 0.25) (layer "F.Cu") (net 23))
 (segment (start 82.55 77.47) (end 83.454357 78.374357) (width 0.25) (layer "F.Cu") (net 23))
 (segment (start 92.490375 74.709357) (end 98.206771 74.709357) (width 0.25) (layer "F.Cu") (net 23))
 (segment (start 98.672762 78.374357) (end 99.77108 77.276039) (width 0.25) (layer "F.Cu") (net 23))
 (segment (start 91.355814 73.574796) (end 92.490375 74.709357) (width 0.25) (layer "F.Cu") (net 23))
 (segment (start 80.01 72.39) (end 81.185 71.215) (width 0.25) (layer "F.Cu") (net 23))
 (segment (start 81.185 71.215) (end 84.519609 71.215) (width 0.25) (layer "F.Cu") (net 23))
 (segment (start 86.885474 73.580865) (end 90.078727 73.580865) (width 0.25) (layer "F.Cu") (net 23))
 (segment (start 99.77108 77.276039) (end 99.77108 76.273666) (width 0.25) (layer "F.Cu") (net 23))
 (segment (start 99.77108 76.273666) (end 98.206771 74.709357) (width 0.25) (layer "F.Cu") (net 23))
 (segment (start 90.078727 73.580865) (end 90.084796 73.574796) (width 0.25) (layer "F.Cu") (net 23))
 (segment (start 86.662709 76.124357) (end 97.081771 76.124357) (width 0.25) (layer "F.Cu") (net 22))
 (segment (start 86.572601 76.034249) (end 86.662709 76.124357) (width 0.25) (layer "F.Cu") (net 22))
 (segment (start 97.081771 76.124357) (end 98.206771 77.249357) (width 0.25) (layer "F.Cu") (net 22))
 (via (at 86.572601 76.034249) (size 0.8) (drill 0.4) (layers "F.Cu" "B.Cu") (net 22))
 (segment (start 84.804572 62.822871) (end 83.036701 61.055) (width 0.25) (layer "B.Cu") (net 22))
 (segment (start 83.036701 61.055) (end 81.375 61.055) (width 0.25) (layer "B.Cu") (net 22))
 (segment (start 86.572601 76.034249) (end 84.365 73.826648) (width 0.25) (layer "B.Cu") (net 22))
 (segment (start 80.01 59.69) (end 82.55 57.15) (width 0.25) (layer "B.Cu") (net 22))
 (segment (start 84.365 71.845) (end 84.804572 71.405428) (width 0.25) (layer "B.Cu") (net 22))
 (segment (start 81.375 61.055) (end 80.01 59.69) (width 0.25) (layer "B.Cu") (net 22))
 (segment (start 84.804572 71.405428) (end 84.804572 62.822871) (width 0.25) (layer "B.Cu") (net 22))
 (segment (start 84.365 73.826648) (end 84.365 71.845) (width 0.25) (layer "B.Cu") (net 22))
 (segment (start 82.55 74.93) (end 90.366128 74.93) (width 0.25) (layer "F.Cu") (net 17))
 (segment (start 90.366128 74.93) (end 90.586771 74.709357) (width 0.25) (layer "F.Cu") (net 17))
 (segment (start 88.046771 49.309357) (end 90.586771 49.309357) (width 0.25) (layer "B.Cu") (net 5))
 (segment (start 101.733269 58.838795) (end 99.599405 60.972659) (width 0.25) (layer "B.Cu") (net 7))
 (segment (start 105.41 71.12) (end 98.839357 64.549357) (width 0.25) (layer "B.Cu") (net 7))
 (segment (start 109.899958 78.972982) (end 105.41 74.483024) (width 0.25) (layer "B.Cu") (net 7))
 (segment (start 99.599405 63.156723) (end 98.206771 64.549357) (width 0.25) (layer "B.Cu") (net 7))
 (segment (start 105.41 74.483024) (end 105.41 71.12) (width 0.25) (layer "B.Cu") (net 7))
 (segment (start 99.599405 60.972659) (end 99.599405 63.156723) (width 0.25) (layer "B.Cu") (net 7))
 (segment (start 98.839357 64.549357) (end 98.206771 64.549357) (width 0.25) (layer "B.Cu") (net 7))
 (segment (start 98.206771 67.089357) (end 99.783945 67.089357) (width 0.25) (layer "F.Cu") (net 8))
 (segment (start 99.783945 67.089357) (end 101.667111 68.972523) (width 0.25) (layer "F.Cu") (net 8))
 (segment (start 102.180935 69.486347) (end 101.667111 68.972523) (width 0.25) (layer "B.Cu") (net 8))
 (segment (start 102.180935 78.873959) (end 102.180935 69.486347) (width 0.25) (layer "B.Cu") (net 8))
 (segment (start 102.279958 78.972982) (end 102.180935 78.873959) (width 0.25) (layer "B.Cu") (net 8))
 (segment (start 81.421522 50.8) (end 81.28 50.8) (width 0.25) (layer "F.Cu") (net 9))
 (segment (start 89.537414 50.8) (end 81.421522 50.8) (width 0.25) (layer "F.Cu") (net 9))
 (segment (start 81.28 50.8) (end 81.408752 50.81277) (width 0.25) (layer "F.Cu") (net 9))
 (segment (start 90.586771 51.849357) (end 89.537414 50.8) (width 0.25) (layer "F.Cu") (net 9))
 (via (at 81.28 50.8) (size 0.8) (drill 0.4) (layers "F.Cu" "B.Cu") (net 9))
 (segment (start 81.28 50.8) (end 81.28 55.88) (width 0.25) (layer "B.Cu") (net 9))
 (segment (start 81.28 55.88) (end 80.01 57.15) (width 0.25) (layer "B.Cu") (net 9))
 (segment (start 91.223167 67.089357) (end 90.586771 67.089357) (width 0.25) (layer "F.Cu") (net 1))
 (segment (start 80.01 50.009941) (end 80.01 52.07) (width 0.25) (layer "F.Cu") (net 1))
 (segment (start 91.055547 47.528133) (end 82.491808 47.528133) (width 0.25) (layer "F.Cu") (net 1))
 (segment (start 95.25 82.55) (end 96.154357 83.454357) (width 0.25) (layer "F.Cu") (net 1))
 (segment (start 99.338141 51.849357) (end 102.356445 48.831053) (width 0.25) (layer "F.Cu") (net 1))
 (segment (start 93.98 83.82) (end 95.25 82.55) (width 0.25) (layer "F.Cu") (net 1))
 (segment (start 98.206771 51.849357) (end 99.338141 51.849357) (width 0.25) (layer "F.Cu") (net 1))
 (segment (start 99.00677 72.969356) (end 102.019569 72.969356) (width 0.25) (layer "F.Cu") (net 1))
 (segment (start 96.154357 83.454357) (end 102.878583 83.454357) (width 0.25) (layer "F.Cu") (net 1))
 (segment (start 102.356445 48.831053) (end 103.029426 48.831053) (width 0.25) (layer "F.Cu") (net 1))
 (segment (start 106.067451 59.76057) (end 107.408021 58.42) (width 0.25) (layer "F.Cu") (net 1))
 (segment (start 106.067451 68.311195) (end 106.067451 59.76057) (width 0.25) (layer "F.Cu") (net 1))
 (segment (start 98.346497 72.029631) (end 98.206771 72.169357) (width 0.25) (layer "F.Cu") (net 1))
 (segment (start 98.206771 72.169357) (end 99.00677 72.969356) (width 0.25) (layer "F.Cu") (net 1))
 (segment (start 88.046771 82.289357) (end 89.577414 83.82) (width 0.25) (layer "F.Cu") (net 1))
 (segment (start 106.067451 68.921474) (end 106.067451 68.311195) (width 0.25) (layer "F.Cu") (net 1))
 (segment (start 91.44 83.82) (end 93.98 83.82) (width 0.25) (layer "F.Cu") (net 1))
 (segment (start 98.206771 51.849357) (end 95.376771 51.849357) (width 0.25) (layer "F.Cu") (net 1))
 (segment (start 102.878583 83.454357) (end 107.359958 78.972982) (width 0.25) (layer "F.Cu") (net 1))
 (segment (start 95.376771 51.849357) (end 91.055547 47.528133) (width 0.25) (layer "F.Cu") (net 1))
 (segment (start 102.019569 72.969356) (end 103.305935 71.68299) (width 0.25) (layer "F.Cu") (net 1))
 (segment (start 82.491808 47.528133) (end 80.01 50.009941) (width 0.25) (layer "F.Cu") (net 1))
 (segment (start 89.577414 83.82) (end 91.44 83.82) (width 0.25) (layer "F.Cu") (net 1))
 (segment (start 103.305935 71.68299) (end 106.067451 68.921474) (width 0.25) (layer "F.Cu") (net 1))
 (via (at 95.25 82.55) (size 0.8) (drill 0.4) (layers "F.Cu" "B.Cu") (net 1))
 (segment (start 85.09 59.205047) (end 87.7161 61.831147) (width 0.25) (layer "B.Cu") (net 1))
 (segment (start 84.337829 50.047829) (end 85.09 50.8) (width 0.25) (layer "B.Cu") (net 1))
 (segment (start 93.126771 67.089357) (end 90.586771 67.089357) (width 0.25) (layer "B.Cu") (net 1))
 (segment (start 85.09 50.8) (end 85.09 59.205047) (width 0.25) (layer "B.Cu") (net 1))
 (segment (start 97.948211 51.849357) (end 95.788258 54.00931) (width 0.25) (layer "B.Cu") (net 1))
 (segment (start 95.25 69.212586) (end 93.126771 67.089357) (width 0.25) (layer "B.Cu") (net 1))
 (segment (start 107.408021 53.217542) (end 108.555563 52.07) (width 0.25) (layer "B.Cu") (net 1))
 (segment (start 103.029426 48.831053) (end 105.316616 48.831053) (width 0.25) (layer "B.Cu") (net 1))
 (segment (start 105.316616 48.831053) (end 108.555563 52.07) (width 0.25) (layer "B.Cu") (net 1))
 (segment (start 80.787711 50.047829) (end 84.337829 50.047829) (width 0.25) (layer "B.Cu") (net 1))
 (segment (start 80.01 52.07) (end 80.01 50.82554) (width 0.25) (layer "B.Cu") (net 1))
 (segment (start 98.206771 72.169357) (end 95.25 69.212586) (width 0.25) (layer "B.Cu") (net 1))
 (segment (start 95.25 82.55) (end 95.25 75.126128) (width 0.25) (layer "B.Cu") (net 1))
 (segment (start 95.788258 54.00931) (end 95.788258 64.231742) (width 0.25) (layer "B.Cu") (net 1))
 (segment (start 93.126771 66.893229) (end 93.126771 67.089357) (width 0.25) (layer "B.Cu") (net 1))
 (segment (start 95.788258 64.231742) (end 93.126771 66.893229) (width 0.25) (layer "B.Cu") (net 1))
 (segment (start 80.01 50.82554) (end 80.787711 50.047829) (width 0.25) (layer "B.Cu") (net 1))
 (segment (start 95.25 75.126128) (end 98.206771 72.169357) (width 0.25) (layer "B.Cu") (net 1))
 (segment (start 107.408021 58.42) (end 107.408021 53.217542) (width 0.25) (layer "B.Cu") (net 1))
 (segment (start 98.206771 51.849357) (end 97.948211 51.849357) (width 0.25) (layer "B.Cu") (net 1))
 (segment (start 110.49 64.77) (end 110.667451 64.947451) (width 0.25) (layer "F.Cu") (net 4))
 (segment (start 110.667451 73.125489) (end 110.667451 68.311195) (width 0.25) (layer "F.Cu") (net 4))
 (segment (start 104.819958 78.972982) (end 110.667451 73.125489) (width 0.25) (layer "F.Cu") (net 4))
 (segment (start 110.667451 64.947451) (end 110.667451 68.311195) (width 0.25) (layer "F.Cu") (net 4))
 (via (at 110.49 64.77) (size 0.8) (drill 0.4) (layers "F.Cu" "B.Cu") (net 4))
 (segment (start 101.667111 61.352523) (end 107.072523 61.352523) (width 0.25) (layer "B.Cu") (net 4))
 (segment (start 107.072523 61.352523) (end 110.49 64.77) (width 0.25) (layer "B.Cu") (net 4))
 (segment (start 104.14 53.625526) (end 104.14 58.879634) (width 0.25) (layer "B.Cu") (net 4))
 (segment (start 104.14 58.879634) (end 101.667111 61.352523) (width 0.25) (layer "B.Cu") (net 4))
 (segment (start 101.733269 51.218795) (end 104.14 53.625526) (width 0.25) (layer "B.Cu") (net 4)))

